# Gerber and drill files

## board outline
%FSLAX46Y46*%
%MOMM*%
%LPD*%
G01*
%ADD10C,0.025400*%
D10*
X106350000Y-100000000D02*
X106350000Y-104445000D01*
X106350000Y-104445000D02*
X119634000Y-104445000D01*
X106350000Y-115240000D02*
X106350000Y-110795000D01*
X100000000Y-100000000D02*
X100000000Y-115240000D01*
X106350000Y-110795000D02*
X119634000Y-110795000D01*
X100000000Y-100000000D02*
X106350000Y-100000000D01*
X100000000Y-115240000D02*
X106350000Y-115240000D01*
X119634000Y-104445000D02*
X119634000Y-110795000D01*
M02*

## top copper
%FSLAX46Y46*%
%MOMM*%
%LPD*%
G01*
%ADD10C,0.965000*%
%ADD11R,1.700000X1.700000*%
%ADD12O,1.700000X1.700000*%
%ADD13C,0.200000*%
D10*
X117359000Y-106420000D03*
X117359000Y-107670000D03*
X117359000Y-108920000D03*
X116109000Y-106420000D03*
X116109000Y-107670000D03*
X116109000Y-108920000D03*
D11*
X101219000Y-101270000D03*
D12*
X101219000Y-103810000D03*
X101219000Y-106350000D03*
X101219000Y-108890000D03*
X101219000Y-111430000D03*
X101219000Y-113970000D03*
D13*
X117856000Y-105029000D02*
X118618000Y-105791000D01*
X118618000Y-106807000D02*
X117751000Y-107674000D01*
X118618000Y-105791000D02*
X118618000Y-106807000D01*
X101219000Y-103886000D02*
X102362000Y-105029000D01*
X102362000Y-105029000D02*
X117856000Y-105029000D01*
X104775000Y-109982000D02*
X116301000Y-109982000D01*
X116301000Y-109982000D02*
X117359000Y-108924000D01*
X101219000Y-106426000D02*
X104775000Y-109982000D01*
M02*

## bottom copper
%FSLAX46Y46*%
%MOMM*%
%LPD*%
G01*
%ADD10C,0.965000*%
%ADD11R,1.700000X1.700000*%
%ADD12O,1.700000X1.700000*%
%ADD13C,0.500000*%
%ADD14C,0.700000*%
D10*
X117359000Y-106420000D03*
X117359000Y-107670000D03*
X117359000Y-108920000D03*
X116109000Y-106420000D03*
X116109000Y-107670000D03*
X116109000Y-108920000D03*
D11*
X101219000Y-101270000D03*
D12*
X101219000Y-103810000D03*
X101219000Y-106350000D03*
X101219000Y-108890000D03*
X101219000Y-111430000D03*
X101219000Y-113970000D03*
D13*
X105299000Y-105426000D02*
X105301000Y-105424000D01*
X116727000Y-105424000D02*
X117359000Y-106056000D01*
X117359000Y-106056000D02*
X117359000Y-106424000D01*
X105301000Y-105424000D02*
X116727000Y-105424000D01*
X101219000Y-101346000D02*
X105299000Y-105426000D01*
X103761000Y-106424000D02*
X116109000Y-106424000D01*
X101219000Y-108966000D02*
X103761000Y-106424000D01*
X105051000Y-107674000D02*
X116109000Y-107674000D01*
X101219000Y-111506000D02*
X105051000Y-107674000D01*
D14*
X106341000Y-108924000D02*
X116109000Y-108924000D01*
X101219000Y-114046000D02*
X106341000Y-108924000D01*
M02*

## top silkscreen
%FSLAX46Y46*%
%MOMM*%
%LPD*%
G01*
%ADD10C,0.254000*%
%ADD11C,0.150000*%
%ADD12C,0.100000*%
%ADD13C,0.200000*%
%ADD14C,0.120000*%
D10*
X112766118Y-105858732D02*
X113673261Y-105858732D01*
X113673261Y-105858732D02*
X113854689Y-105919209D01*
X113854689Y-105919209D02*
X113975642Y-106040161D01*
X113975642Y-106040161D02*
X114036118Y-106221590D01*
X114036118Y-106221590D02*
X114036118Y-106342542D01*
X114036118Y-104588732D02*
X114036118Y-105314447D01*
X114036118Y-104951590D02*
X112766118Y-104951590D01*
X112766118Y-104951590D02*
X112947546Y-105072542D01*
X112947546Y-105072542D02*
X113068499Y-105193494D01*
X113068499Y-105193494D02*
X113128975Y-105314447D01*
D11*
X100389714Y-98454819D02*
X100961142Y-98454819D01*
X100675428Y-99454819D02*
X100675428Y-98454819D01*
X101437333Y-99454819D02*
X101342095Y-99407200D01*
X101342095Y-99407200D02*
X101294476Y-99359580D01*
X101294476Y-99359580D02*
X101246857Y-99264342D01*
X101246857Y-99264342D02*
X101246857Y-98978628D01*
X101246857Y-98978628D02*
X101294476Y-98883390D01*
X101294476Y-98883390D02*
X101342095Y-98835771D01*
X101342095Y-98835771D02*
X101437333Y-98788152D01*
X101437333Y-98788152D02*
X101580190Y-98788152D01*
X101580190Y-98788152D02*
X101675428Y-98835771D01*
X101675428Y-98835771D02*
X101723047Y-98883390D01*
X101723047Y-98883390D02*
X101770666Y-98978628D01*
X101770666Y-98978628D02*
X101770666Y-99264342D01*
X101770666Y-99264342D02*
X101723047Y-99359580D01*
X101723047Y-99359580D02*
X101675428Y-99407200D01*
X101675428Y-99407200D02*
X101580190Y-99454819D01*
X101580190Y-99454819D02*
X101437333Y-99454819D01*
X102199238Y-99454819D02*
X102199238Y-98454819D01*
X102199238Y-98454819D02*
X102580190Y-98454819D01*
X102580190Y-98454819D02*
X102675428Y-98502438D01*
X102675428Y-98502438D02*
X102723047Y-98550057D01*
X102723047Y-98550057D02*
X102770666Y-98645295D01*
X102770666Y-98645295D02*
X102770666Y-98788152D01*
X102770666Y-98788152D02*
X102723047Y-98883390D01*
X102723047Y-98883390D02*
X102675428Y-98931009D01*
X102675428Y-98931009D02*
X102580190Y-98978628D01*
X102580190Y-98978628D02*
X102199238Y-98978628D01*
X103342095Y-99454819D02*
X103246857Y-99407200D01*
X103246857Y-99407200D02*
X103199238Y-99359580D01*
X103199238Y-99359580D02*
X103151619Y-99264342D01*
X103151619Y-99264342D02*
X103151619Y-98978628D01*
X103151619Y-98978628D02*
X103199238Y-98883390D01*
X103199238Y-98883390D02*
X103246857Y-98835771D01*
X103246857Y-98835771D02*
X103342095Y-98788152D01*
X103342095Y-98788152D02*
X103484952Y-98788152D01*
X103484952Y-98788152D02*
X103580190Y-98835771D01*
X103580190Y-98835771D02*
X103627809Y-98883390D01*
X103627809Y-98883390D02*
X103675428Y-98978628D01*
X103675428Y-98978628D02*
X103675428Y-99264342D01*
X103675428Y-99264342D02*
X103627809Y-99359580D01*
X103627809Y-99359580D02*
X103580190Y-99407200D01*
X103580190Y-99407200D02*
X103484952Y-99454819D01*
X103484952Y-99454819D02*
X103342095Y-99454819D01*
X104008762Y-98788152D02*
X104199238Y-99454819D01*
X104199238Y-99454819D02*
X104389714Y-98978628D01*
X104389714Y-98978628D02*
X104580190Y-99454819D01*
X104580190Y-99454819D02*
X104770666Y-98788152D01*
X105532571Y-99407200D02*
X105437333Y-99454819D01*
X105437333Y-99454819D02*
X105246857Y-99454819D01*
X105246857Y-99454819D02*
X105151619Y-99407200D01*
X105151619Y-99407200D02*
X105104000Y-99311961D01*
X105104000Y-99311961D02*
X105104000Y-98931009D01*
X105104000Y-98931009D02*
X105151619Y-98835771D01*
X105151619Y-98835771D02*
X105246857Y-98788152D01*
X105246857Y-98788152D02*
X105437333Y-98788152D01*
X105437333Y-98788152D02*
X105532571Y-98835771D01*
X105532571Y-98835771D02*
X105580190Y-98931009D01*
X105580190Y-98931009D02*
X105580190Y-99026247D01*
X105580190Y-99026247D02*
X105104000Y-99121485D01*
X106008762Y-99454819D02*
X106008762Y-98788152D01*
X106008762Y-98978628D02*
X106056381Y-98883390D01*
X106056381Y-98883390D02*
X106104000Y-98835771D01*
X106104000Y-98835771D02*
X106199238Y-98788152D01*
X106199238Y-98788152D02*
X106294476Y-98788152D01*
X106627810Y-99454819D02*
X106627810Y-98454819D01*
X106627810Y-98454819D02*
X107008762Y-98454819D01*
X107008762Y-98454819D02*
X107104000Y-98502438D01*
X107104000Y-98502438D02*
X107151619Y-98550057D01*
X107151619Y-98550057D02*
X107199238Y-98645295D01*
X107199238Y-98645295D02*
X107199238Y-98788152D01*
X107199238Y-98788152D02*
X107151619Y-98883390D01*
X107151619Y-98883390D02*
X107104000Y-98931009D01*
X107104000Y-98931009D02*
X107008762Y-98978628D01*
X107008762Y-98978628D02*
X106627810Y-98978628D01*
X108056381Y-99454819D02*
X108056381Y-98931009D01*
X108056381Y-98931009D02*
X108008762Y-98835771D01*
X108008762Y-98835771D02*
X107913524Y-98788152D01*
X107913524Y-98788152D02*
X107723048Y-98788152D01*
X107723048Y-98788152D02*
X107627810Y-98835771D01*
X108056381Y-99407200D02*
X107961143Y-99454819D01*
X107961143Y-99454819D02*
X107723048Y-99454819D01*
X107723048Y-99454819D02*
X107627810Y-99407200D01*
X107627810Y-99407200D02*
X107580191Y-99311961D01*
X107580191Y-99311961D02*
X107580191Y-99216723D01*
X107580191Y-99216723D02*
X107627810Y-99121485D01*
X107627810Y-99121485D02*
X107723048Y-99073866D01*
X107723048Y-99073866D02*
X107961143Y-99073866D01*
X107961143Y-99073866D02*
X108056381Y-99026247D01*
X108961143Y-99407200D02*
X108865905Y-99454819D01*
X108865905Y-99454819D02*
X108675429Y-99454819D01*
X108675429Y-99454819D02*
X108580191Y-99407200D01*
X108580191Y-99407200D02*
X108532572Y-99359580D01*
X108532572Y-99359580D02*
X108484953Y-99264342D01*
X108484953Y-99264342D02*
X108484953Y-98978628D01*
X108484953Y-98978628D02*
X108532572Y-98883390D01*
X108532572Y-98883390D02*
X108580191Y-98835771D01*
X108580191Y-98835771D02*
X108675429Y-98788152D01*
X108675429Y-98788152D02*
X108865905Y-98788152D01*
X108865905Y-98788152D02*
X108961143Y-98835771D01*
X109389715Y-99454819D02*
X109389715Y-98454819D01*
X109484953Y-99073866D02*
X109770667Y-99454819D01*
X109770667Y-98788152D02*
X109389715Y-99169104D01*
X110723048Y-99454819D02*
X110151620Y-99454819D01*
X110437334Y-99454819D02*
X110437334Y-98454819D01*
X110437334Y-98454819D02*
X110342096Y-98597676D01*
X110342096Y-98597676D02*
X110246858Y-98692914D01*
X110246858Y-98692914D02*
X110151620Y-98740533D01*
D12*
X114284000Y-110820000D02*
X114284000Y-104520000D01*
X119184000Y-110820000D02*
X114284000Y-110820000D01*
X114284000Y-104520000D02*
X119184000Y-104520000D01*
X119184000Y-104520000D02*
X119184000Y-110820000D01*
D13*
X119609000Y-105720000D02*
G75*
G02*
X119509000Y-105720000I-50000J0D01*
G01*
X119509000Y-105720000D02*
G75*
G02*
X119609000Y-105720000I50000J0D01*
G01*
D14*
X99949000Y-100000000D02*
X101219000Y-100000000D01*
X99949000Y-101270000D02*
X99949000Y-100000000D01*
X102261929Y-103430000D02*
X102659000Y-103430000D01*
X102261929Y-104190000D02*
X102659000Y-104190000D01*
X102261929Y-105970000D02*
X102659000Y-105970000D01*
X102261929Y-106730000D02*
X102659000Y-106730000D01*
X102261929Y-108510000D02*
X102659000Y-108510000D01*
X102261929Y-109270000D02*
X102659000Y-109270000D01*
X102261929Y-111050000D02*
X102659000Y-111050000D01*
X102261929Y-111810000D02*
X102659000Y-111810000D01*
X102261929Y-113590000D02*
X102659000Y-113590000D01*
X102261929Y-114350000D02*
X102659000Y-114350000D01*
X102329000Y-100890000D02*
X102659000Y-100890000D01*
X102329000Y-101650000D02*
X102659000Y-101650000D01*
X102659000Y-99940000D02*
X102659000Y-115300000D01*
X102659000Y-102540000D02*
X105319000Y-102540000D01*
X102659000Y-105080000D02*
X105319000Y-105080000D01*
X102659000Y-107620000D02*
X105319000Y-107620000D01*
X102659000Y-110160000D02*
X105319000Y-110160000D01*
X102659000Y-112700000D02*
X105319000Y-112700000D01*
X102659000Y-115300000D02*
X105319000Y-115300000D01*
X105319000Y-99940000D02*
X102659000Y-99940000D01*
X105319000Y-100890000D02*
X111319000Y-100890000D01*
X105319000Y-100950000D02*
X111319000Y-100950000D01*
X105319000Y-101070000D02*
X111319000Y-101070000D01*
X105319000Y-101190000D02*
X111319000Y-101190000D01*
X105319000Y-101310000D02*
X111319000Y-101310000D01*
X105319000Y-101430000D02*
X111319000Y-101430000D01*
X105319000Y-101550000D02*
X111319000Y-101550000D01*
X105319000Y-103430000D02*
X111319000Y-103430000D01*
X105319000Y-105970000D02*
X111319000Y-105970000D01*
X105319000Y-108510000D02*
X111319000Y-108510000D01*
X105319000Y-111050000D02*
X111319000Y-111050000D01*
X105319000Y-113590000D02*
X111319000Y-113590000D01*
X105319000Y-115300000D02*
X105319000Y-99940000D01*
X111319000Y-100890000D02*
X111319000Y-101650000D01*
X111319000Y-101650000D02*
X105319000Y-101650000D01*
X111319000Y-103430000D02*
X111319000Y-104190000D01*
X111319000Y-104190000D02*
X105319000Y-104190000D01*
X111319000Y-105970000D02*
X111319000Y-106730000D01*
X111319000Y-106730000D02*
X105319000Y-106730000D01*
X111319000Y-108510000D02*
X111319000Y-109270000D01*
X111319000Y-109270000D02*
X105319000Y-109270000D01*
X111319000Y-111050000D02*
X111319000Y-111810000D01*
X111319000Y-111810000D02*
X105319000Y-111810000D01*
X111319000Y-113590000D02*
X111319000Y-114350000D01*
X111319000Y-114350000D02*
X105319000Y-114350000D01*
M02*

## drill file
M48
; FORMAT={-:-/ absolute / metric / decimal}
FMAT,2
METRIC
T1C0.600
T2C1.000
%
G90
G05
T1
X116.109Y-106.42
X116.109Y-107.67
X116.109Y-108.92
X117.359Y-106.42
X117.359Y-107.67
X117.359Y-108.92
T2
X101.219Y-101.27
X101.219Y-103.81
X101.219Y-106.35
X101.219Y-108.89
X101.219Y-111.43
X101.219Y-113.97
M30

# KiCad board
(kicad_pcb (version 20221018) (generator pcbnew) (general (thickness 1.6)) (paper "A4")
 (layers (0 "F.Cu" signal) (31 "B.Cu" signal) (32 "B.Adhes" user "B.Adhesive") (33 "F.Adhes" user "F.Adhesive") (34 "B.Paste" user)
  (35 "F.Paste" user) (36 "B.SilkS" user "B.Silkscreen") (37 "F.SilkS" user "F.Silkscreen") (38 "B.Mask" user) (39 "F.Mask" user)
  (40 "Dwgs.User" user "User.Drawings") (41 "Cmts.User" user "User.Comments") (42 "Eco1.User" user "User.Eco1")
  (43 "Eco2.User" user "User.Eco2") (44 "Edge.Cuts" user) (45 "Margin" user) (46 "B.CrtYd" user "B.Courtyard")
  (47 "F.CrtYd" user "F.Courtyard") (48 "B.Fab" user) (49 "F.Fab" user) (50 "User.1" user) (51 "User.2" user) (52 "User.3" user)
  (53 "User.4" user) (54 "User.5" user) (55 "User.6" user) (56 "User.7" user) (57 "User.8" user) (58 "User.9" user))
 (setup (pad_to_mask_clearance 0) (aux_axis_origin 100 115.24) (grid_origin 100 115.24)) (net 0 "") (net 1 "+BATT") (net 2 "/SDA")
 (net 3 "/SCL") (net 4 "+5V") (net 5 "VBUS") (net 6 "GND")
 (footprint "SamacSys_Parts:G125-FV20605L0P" (layer "F.Cu") (at 117.359 106.42 90)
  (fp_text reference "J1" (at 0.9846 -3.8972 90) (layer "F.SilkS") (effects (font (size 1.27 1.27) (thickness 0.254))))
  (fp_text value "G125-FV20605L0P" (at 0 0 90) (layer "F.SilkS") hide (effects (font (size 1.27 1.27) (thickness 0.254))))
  (fp_line (start -4.4 -3.075) (end 1.9 -3.075) (stroke (width 0.1) (type solid)) (layer "F.SilkS"))
  (fp_line (start -4.4 1.825) (end -4.4 -3.075) (stroke (width 0.1) (type solid)) (layer "F.SilkS"))
  (fp_line (start 1.9 -3.075) (end 1.9 1.825) (stroke (width 0.1) (type solid)) (layer "F.SilkS"))
  (fp_line (start 1.9 1.825) (end -4.4 1.825) (stroke (width 0.1) (type solid)) (layer "F.SilkS"))
  (fp_circle (center 0.7 2.2) (end 0.7 2.25) (stroke (width 0.2) (type solid)) (fill none) (layer "F.SilkS"))
  (pad "1" thru_hole circle (at 0 0 90) (size 0.965 0.965) (drill 0.6) (layers "*.Cu" "*.Mask") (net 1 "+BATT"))
  (pad "2" thru_hole circle (at -1.25 0 90) (size 0.965 0.965) (drill 0.6) (layers "*.Cu" "*.Mask") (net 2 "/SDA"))
  (pad "3" thru_hole circle (at -2.5 0 90) (size 0.965 0.965) (drill 0.6) (layers "*.Cu" "*.Mask") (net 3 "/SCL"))
  (pad "4" thru_hole circle (at 0 -1.25 90) (size 0.965 0.965) (drill 0.6) (layers "*.Cu" "*.Mask") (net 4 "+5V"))
  (pad "5" thru_hole circle (at -1.25 -1.25 90) (size 0.965 0.965) (drill 0.6) (layers "*.Cu" "*.Mask") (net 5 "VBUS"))
  (pad "6" thru_hole circle (at -2.5 -1.25 90) (size 0.965 0.965) (drill 0.6) (layers "*.Cu" "*.Mask") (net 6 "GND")))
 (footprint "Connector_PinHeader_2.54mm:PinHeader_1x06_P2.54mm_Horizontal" (layer "F.Cu") (at 101.219 101.27)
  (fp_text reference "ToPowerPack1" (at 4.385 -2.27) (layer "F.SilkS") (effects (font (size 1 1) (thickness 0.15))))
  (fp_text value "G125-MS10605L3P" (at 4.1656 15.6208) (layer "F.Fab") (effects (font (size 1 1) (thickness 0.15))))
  (fp_line (start -1.27 -1.27) (end 0 -1.27) (stroke (width 0.12) (type solid)) (layer "F.SilkS"))
  (fp_line (start -1.27 0) (end -1.27 -1.27) (stroke (width 0.12) (type solid)) (layer "F.SilkS"))
  (fp_line (start 1.042929 2.16) (end 1.44 2.16) (stroke (width 0.12) (type solid)) (layer "F.SilkS"))
  (fp_line (start 1.042929 2.92) (end 1.44 2.92) (stroke (width 0.12) (type solid)) (layer "F.SilkS"))
  (fp_line (start 1.042929 4.7) (end 1.44 4.7) (stroke (width 0.12) (type solid)) (layer "F.SilkS"))
  (fp_line (start 1.042929 5.46) (end 1.44 5.46) (stroke (width 0.12) (type solid)) (layer "F.SilkS"))
  (fp_line (start 1.042929 7.24) (end 1.44 7.24) (stroke (width 0.12) (type solid)) (layer "F.SilkS"))
  (fp_line (start 1.042929 8) (end 1.44 8) (stroke (width 0.12) (type solid)) (layer "F.SilkS"))
  (fp_line (start 1.042929 9.78) (end 1.44 9.78) (stroke (width 0.12) (type solid)) (layer "F.SilkS"))
  (fp_line (start 1.042929 10.54) (end 1.44 10.54) (stroke (width 0.12) (type solid)) (layer "F.SilkS"))
  (fp_line (start 1.042929 12.32) (end 1.44 12.32) (stroke (width 0.12) (type solid)) (layer "F.SilkS"))
  (fp_line (start 1.042929 13.08) (end 1.44 13.08) (stroke (width 0.12) (type solid)) (layer "F.SilkS"))
  (fp_line (start 1.11 -0.38) (end 1.44 -0.38) (stroke (width 0.12) (type solid)) (layer "F.SilkS"))
  (fp_line (start 1.11 0.38) (end 1.44 0.38) (stroke (width 0.12) (type solid)) (layer "F.SilkS"))
  (fp_line (start 1.44 -1.33) (end 1.44 14.03) (stroke (width 0.12) (type solid)) (layer "F.SilkS"))
  (fp_line (start 1.44 1.27) (end 4.1 1.27) (stroke (width 0.12) (type solid)) (layer "F.SilkS"))
  (fp_line (start 1.44 3.81) (end 4.1 3.81) (stroke (width 0.12) (type solid)) (layer "F.SilkS"))
  (fp_line (start 1.44 6.35) (end 4.1 6.35) (stroke (width 0.12) (type solid)) (layer "F.SilkS"))
  (fp_line (start 1.44 8.89) (end 4.1 8.89) (stroke (width 0.12) (type solid)) (layer "F.SilkS"))
  (fp_line (start 1.44 11.43) (end 4.1 11.43) (stroke (width 0.12) (type solid)) (layer "F.SilkS"))
  (fp_line (start 1.44 14.03) (end 4.1 14.03) (stroke (width 0.12) (type solid)) (layer "F.SilkS"))
  (fp_line (start 4.1 -1.33) (end 1.44 -1.33) (stroke (width 0.12) (type solid)) (layer "F.SilkS"))
  (fp_line (start 4.1 -0.38) (end 10.1 -0.38) (stroke (width 0.12) (type solid)) (layer "F.SilkS"))
  (fp_line (start 4.1 -0.32) (end 10.1 -0.32) (stroke (width 0.12) (type solid)) (layer "F.SilkS"))
  (fp_line (start 4.1 -0.2) (end 10.1 -0.2) (stroke (width 0.12) (type solid)) (layer "F.SilkS"))
  (fp_line (start 4.1 -0.08) (end 10.1 -0.08) (stroke (width 0.12) (type solid)) (layer "F.SilkS"))
  (fp_line (start 4.1 0.04) (end 10.1 0.04) (stroke (width 0.12) (type solid)) (layer "F.SilkS"))
  (fp_line (start 4.1 0.16) (end 10.1 0.16) (stroke (width 0.12) (type solid)) (layer "F.SilkS"))
  (fp_line (start 4.1 0.28) (end 10.1 0.28) (stroke (width 0.12) (type solid)) (layer "F.SilkS"))
  (fp_line (start 4.1 2.16) (end 10.1 2.16) (stroke (width 0.12) (type solid)) (layer "F.SilkS"))
  (fp_line (start 4.1 4.7) (end 10.1 4.7) (stroke (width 0.12) (type solid)) (layer "F.SilkS"))
  (fp_line (start 4.1 7.24) (end 10.1 7.24) (stroke (width 0.12) (type solid)) (layer "F.SilkS"))
  (fp_line (start 4.1 9.78) (end 10.1 9.78) (stroke (width 0.12) (type solid)) (layer "F.SilkS"))
  (fp_line (start 4.1 12.32) (end 10.1 12.32) (stroke (width 0.12) (type solid)) (layer "F.SilkS"))
  (fp_line (start 4.1 14.03) (end 4.1 -1.33) (stroke (width 0.12) (type solid)) (layer "F.SilkS"))
  (fp_line (start 10.1 -0.38) (end 10.1 0.38) (stroke (width 0.12) (type solid)) (layer "F.SilkS"))
  (fp_line (start 10.1 0.38) (end 4.1 0.38) (stroke (width 0.12) (type solid)) (layer "F.SilkS"))
  (fp_line (start 10.1 2.16) (end 10.1 2.92) (stroke (width 0.12) (type solid)) (layer "F.SilkS"))
  (fp_line (start 10.1 2.92) (end 4.1 2.92) (stroke (width 0.12) (type solid)) (layer "F.SilkS"))
  (fp_line (start 10.1 4.7) (end 10.1 5.46) (stroke (width 0.12) (type solid)) (layer "F.SilkS"))
  (fp_line (start 10.1 5.46) (end 4.1 5.46) (stroke (width 0.12) (type solid)) (layer "F.SilkS"))
  (fp_line (start 10.1 7.24) (end 10.1 8) (stroke (width 0.12) (type solid)) (layer "F.SilkS"))
  (fp_line (start 10.1 8) (end 4.1 8) (stroke (width 0.12) (type solid)) (layer "F.SilkS"))
  (fp_line (start 10.1 9.78) (end 10.1 10.54) (stroke (width 0.12) (type solid)) (layer "F.SilkS"))
  (fp_line (start 10.1 10.54) (end 4.1 10.54) (stroke (width 0.12) (type solid)) (layer "F.SilkS"))
  (fp_line (start 10.1 12.32) (end 10.1 13.08) (stroke (width 0.12) (type solid)) (layer "F.SilkS"))
  (fp_line (start 10.1 13.08) (end 4.1 13.08) (stroke (width 0.12) (type solid)) (layer "F.SilkS"))
  (pad "1" thru_hole rect (at 0 0) (size 1.7 1.7) (drill 1) (layers "*.Cu" "*.Mask") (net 1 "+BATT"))
  (pad "2" thru_hole oval (at 0 2.54) (size 1.7 1.7) (drill 1) (layers "*.Cu" "*.Mask") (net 2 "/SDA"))
  (pad "3" thru_hole oval (at 0 5.08) (size 1.7 1.7) (drill 1) (layers "*.Cu" "*.Mask") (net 3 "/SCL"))
  (pad "4" thru_hole oval (at 0 7.62) (size 1.7 1.7) (drill 1) (layers "*.Cu" "*.Mask") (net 4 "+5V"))
  (pad "5" thru_hole oval (at 0 10.16) (size 1.7 1.7) (drill 1) (layers "*.Cu" "*.Mask") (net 5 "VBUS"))
  (pad "6" thru_hole oval (at 0 12.7) (size 1.7 1.7) (drill 1) (layers "*.Cu" "*.Mask") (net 6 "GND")))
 (gr_line (start 106.35 100) (end 106.35 104.445) (stroke (width 0.0254) (type default)) (layer "Edge.Cuts"))
 (gr_line (start 106.35 104.445) (end 119.634 104.445) (stroke (width 0.0254) (type default)) (layer "Edge.Cuts"))
 (gr_line (start 106.35 115.24) (end 106.35 110.795) (stroke (width 0.0254) (type default)) (layer "Edge.Cuts"))
 (gr_line (start 100 100) (end 100 115.24) (stroke (width 0.0254) (type default)) (layer "Edge.Cuts"))
 (gr_line (start 106.35 110.795) (end 119.634 110.795) (stroke (width 0.0254) (type default)) (layer "Edge.Cuts"))
 (gr_line (start 100 100) (end 106.35 100) (stroke (width 0.0254) (type default)) (layer "Edge.Cuts"))
 (gr_line (start 100 115.24) (end 106.35 115.24) (stroke (width 0.0254) (type default)) (layer "Edge.Cuts"))
 (gr_line (start 119.634 104.445) (end 119.634 110.795) (stroke (width 0.0254) (type default)) (layer "Edge.Cuts"))
 (segment (start 105.299 105.426) (end 105.301 105.424) (width 0.5) (layer "B.Cu") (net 1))
 (segment (start 116.727 105.424) (end 117.359 106.056) (width 0.5) (layer "B.Cu") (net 1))
 (segment (start 117.359 106.056) (end 117.359 106.424) (width 0.5) (layer "B.Cu") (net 1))
 (segment (start 105.301 105.424) (end 116.727 105.424) (width 0.5) (layer "B.Cu") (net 1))
 (segment (start 101.219 101.346) (end 105.299 105.426) (width 0.5) (layer "B.Cu") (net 1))
 (segment (start 117.856 105.029) (end 118.618 105.791) (width 0.2) (layer "F.Cu") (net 2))
 (segment (start 118.618 106.807) (end 117.751 107.674) (width 0.2) (layer "F.Cu") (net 2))
 (segment (start 118.618 105.791) (end 118.618 106.807) (width 0.2) (layer "F.Cu") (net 2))
 (segment (start 101.219 103.886) (end 102.362 105.029) (width 0.2) (layer "F.Cu") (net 2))
 (segment (start 102.362 105.029) (end 117.856 105.029) (width 0.2) (layer "F.Cu") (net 2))
 (segment (start 104.775 109.982) (end 116.301 109.982) (width 0.2) (layer "F.Cu") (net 3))
 (segment (start 116.301 109.982) (end 117.359 108.924) (width 0.2) (layer "F.Cu") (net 3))
 (segment (start 101.219 106.426) (end 104.775 109.982) (width 0.2) (layer "F.Cu") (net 3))
 (segment (start 103.761 106.424) (end 116.109 106.424) (width 0.5) (layer "B.Cu") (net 4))
 (segment (start 101.219 108.966) (end 103.761 106.424) (width 0.5) (layer "B.Cu") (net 4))
 (segment (start 105.051 107.674) (end 116.109 107.674) (width 0.5) (layer "B.Cu") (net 5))
 (segment (start 101.219 111.506) (end 105.051 107.674) (width 0.5) (layer "B.Cu") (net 5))
 (segment (start 106.341 108.924) (end 116.109 108.924) (width 0.7) (layer "B.Cu") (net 6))
 (segment (start 101.219 114.046) (end 106.341 108.924) (width 0.7) (layer "B.Cu") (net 6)))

